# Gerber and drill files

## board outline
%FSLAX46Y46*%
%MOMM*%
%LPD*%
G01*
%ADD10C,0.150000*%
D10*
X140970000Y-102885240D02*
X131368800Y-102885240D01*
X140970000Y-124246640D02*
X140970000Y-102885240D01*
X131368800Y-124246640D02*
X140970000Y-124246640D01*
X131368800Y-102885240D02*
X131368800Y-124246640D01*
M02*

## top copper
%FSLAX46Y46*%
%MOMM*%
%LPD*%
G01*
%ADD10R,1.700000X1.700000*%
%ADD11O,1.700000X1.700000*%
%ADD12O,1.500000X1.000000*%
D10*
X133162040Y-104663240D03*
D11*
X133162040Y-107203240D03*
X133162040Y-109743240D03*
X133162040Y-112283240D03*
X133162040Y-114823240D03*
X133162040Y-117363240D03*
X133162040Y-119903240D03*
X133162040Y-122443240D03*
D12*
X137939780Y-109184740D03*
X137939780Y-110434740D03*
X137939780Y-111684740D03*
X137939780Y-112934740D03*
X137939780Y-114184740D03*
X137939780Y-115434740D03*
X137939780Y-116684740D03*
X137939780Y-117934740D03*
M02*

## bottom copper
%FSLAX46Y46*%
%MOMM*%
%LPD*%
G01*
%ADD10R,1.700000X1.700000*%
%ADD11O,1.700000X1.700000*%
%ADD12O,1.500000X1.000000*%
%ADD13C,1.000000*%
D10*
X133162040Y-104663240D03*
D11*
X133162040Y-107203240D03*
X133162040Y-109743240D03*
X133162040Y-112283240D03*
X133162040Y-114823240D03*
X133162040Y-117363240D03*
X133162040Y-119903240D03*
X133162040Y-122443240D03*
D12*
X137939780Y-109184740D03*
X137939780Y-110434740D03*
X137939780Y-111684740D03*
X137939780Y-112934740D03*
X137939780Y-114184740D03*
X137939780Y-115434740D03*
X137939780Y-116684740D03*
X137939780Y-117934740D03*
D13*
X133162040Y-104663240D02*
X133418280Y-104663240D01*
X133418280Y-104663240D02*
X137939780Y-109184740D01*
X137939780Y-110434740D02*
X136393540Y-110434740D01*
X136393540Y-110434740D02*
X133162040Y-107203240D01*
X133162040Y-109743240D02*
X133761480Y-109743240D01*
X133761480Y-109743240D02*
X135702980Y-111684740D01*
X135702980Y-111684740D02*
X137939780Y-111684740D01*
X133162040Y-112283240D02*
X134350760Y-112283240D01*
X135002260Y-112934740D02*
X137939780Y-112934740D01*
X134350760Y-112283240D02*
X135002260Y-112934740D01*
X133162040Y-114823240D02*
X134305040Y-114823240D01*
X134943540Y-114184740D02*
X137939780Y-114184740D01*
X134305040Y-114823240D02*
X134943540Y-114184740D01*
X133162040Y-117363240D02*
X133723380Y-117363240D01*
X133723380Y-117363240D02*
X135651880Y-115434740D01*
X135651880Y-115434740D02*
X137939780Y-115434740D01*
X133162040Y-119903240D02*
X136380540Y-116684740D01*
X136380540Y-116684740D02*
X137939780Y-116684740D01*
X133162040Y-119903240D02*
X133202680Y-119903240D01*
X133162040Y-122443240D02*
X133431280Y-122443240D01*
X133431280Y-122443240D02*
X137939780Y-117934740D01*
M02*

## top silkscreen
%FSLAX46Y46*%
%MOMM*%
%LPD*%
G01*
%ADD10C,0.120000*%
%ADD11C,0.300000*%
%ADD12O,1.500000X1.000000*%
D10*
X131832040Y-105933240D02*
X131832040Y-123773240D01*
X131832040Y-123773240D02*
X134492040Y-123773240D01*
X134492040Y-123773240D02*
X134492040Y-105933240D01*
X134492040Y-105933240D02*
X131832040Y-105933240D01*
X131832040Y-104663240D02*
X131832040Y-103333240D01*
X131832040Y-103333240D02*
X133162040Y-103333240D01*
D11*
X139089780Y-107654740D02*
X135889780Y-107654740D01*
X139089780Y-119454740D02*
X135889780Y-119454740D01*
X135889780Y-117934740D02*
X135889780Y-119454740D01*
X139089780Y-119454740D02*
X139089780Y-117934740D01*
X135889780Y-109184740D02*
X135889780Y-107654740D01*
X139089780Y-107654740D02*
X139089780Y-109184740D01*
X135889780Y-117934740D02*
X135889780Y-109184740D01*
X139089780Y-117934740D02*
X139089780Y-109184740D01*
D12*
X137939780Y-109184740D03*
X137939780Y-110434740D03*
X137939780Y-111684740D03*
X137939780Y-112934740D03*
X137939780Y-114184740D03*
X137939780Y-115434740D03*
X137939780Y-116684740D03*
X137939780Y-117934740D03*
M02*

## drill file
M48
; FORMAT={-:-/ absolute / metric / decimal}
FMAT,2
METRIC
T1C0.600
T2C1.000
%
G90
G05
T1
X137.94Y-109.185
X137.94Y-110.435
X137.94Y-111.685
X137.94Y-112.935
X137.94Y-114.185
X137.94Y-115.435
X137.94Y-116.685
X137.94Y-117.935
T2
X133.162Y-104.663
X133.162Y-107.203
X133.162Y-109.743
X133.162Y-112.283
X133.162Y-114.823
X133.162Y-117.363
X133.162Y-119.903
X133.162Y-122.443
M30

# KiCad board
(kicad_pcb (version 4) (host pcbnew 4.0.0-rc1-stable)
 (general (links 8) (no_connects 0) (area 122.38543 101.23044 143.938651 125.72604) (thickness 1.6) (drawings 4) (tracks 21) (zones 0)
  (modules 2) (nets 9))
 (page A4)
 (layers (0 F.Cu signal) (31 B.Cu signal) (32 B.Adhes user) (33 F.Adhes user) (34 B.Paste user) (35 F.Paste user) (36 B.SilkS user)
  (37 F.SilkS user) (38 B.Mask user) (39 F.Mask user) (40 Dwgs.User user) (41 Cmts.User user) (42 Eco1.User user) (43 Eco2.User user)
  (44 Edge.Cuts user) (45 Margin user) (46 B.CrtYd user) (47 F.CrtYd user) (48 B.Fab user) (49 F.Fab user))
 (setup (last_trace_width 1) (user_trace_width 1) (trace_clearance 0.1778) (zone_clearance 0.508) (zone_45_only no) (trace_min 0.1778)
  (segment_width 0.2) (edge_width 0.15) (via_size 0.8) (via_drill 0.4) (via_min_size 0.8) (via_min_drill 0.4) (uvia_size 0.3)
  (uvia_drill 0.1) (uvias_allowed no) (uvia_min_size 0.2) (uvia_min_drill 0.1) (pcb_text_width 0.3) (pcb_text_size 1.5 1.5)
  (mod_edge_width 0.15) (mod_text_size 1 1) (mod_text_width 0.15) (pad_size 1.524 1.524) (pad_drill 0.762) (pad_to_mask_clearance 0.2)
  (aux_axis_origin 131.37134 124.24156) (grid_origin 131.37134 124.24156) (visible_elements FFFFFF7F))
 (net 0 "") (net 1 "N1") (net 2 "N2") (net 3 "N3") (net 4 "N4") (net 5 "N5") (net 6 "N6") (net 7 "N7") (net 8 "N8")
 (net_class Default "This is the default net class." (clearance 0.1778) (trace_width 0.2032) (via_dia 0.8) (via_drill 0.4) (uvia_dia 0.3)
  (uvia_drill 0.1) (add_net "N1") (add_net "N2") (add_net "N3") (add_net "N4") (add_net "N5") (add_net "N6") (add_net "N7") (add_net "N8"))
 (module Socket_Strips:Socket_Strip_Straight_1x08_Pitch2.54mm (layer F.Cu) (at 133.16204 104.66324)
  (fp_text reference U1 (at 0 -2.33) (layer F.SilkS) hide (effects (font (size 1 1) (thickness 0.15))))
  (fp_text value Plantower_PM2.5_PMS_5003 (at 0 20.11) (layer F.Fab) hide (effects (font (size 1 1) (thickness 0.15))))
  (fp_line (start -1.33 1.27) (end -1.33 19.11) (layer F.SilkS) (width 0.12))
  (fp_line (start -1.33 19.11) (end 1.33 19.11) (layer F.SilkS) (width 0.12))
  (fp_line (start 1.33 19.11) (end 1.33 1.27) (layer F.SilkS) (width 0.12))
  (fp_line (start 1.33 1.27) (end -1.33 1.27) (layer F.SilkS) (width 0.12))
  (fp_line (start -1.33 0) (end -1.33 -1.33) (layer F.SilkS) (width 0.12))
  (fp_line (start -1.33 -1.33) (end 0 -1.33) (layer F.SilkS) (width 0.12))
  (pad 1 thru_hole rect (at 0 0) (size 1.7 1.7) (drill 1) (layers *.Cu *.Mask) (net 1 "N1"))
  (pad 2 thru_hole oval (at 0 2.54) (size 1.7 1.7) (drill 1) (layers *.Cu *.Mask) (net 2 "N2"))
  (pad 3 thru_hole oval (at 0 5.08) (size 1.7 1.7) (drill 1) (layers *.Cu *.Mask) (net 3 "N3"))
  (pad 4 thru_hole oval (at 0 7.62) (size 1.7 1.7) (drill 1) (layers *.Cu *.Mask) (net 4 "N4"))
  (pad 5 thru_hole oval (at 0 10.16) (size 1.7 1.7) (drill 1) (layers *.Cu *.Mask) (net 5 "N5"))
  (pad 6 thru_hole oval (at 0 12.7) (size 1.7 1.7) (drill 1) (layers *.Cu *.Mask) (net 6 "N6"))
  (pad 7 thru_hole oval (at 0 15.24) (size 1.7 1.7) (drill 1) (layers *.Cu *.Mask) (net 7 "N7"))
  (pad 8 thru_hole oval (at 0 17.78) (size 1.7 1.7) (drill 1) (layers *.Cu *.Mask) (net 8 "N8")))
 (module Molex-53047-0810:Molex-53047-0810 (layer F.Cu) (at 137.93978 117.93474 90)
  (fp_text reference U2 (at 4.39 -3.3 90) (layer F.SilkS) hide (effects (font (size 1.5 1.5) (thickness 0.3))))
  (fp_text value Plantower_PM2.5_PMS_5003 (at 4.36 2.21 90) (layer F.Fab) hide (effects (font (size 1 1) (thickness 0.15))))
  (fp_line (start 10.28 1.15) (end 10.28 -2.05) (layer F.SilkS) (width 0.3))
  (fp_line (start -1.52 1.15) (end -1.52 -2.05) (layer F.SilkS) (width 0.3))
  (fp_line (start 0 -2.05) (end -1.52 -2.05) (layer F.SilkS) (width 0.3))
  (fp_line (start -1.52 1.15) (end 0 1.15) (layer F.SilkS) (width 0.3))
  (fp_line (start 8.75 -2.05) (end 10.28 -2.05) (layer F.SilkS) (width 0.3))
  (fp_line (start 10.28 1.15) (end 8.75 1.15) (layer F.SilkS) (width 0.3))
  (fp_line (start 0 -2.05) (end 8.75 -2.05) (layer F.SilkS) (width 0.3))
  (fp_line (start 0 1.15) (end 8.75 1.15) (layer F.SilkS) (width 0.3))
  (pad 1 thru_hole oval (at 8.75 0 90) (size 1 1.5) (drill 0.6) (layers *.Cu *.Mask F.SilkS) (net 1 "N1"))
  (pad 2 thru_hole oval (at 7.5 0 90) (size 1 1.5) (drill 0.6) (layers *.Cu *.Mask F.SilkS) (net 2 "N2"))
  (pad 3 thru_hole oval (at 6.25 0 90) (size 1 1.5) (drill 0.6) (layers *.Cu *.Mask F.SilkS) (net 3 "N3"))
  (pad 4 thru_hole oval (at 5 0 90) (size 1 1.5) (drill 0.6) (layers *.Cu *.Mask F.SilkS) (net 4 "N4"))
  (pad 5 thru_hole oval (at 3.75 0 90) (size 1 1.5) (drill 0.6) (layers *.Cu *.Mask F.SilkS) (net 5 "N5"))
  (pad 6 thru_hole oval (at 2.5 0 90) (size 1 1.5) (drill 0.6) (layers *.Cu *.Mask F.SilkS) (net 6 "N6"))
  (pad 7 thru_hole oval (at 1.25 0 90) (size 1 1.5) (drill 0.6) (layers *.Cu *.Mask F.SilkS) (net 7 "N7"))
  (pad 8 thru_hole oval (at 0 0 90) (size 1 1.5) (drill 0.6) (layers *.Cu *.Mask F.SilkS) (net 8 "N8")))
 (gr_line (start 140.97 102.88524) (end 131.3688 102.88524) (angle 90) (layer Edge.Cuts) (width 0.15))
 (gr_line (start 140.97 124.24664) (end 140.97 102.88524) (angle 90) (layer Edge.Cuts) (width 0.15))
 (gr_line (start 131.3688 124.24664) (end 140.97 124.24664) (angle 90) (layer Edge.Cuts) (width 0.15))
 (gr_line (start 131.3688 102.88524) (end 131.3688 124.24664) (angle 90) (layer Edge.Cuts) (width 0.15))
 (segment (start 133.16204 104.66324) (end 133.41828 104.66324) (width 1) (layer B.Cu) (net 1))
 (segment (start 133.41828 104.66324) (end 137.93978 109.18474) (width 1) (layer B.Cu) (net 1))
 (segment (start 137.93978 110.43474) (end 136.39354 110.43474) (width 1) (layer B.Cu) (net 2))
 (segment (start 136.39354 110.43474) (end 133.16204 107.20324) (width 1) (layer B.Cu) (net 2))
 (segment (start 133.16204 109.74324) (end 133.76148 109.74324) (width 1) (layer B.Cu) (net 3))
 (segment (start 133.76148 109.74324) (end 135.70298 111.68474) (width 1) (layer B.Cu) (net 3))
 (segment (start 135.70298 111.68474) (end 137.93978 111.68474) (width 1) (layer B.Cu) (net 3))
 (segment (start 133.16204 112.28324) (end 134.35076 112.28324) (width 1) (layer B.Cu) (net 4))
 (segment (start 135.00226 112.93474) (end 137.93978 112.93474) (width 1) (layer B.Cu) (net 4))
 (segment (start 134.35076 112.28324) (end 135.00226 112.93474) (width 1) (layer B.Cu) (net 4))
 (segment (start 133.16204 114.82324) (end 134.30504 114.82324) (width 1) (layer B.Cu) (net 5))
 (segment (start 134.94354 114.18474) (end 137.93978 114.18474) (width 1) (layer B.Cu) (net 5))
 (segment (start 134.30504 114.82324) (end 134.94354 114.18474) (width 1) (layer B.Cu) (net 5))
 (segment (start 133.16204 117.36324) (end 133.72338 117.36324) (width 1) (layer B.Cu) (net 6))
 (segment (start 133.72338 117.36324) (end 135.65188 115.43474) (width 1) (layer B.Cu) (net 6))
 (segment (start 135.65188 115.43474) (end 137.93978 115.43474) (width 1) (layer B.Cu) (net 6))
 (segment (start 133.16204 119.90324) (end 136.38054 116.68474) (width 1) (layer B.Cu) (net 7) (status 400000))
 (segment (start 136.38054 116.68474) (end 137.93978 116.68474) (width 1) (layer B.Cu) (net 7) (status 800000))
 (segment (start 133.16204 119.90324) (end 133.20268 119.90324) (width 1) (layer B.Cu) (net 7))
 (segment (start 133.16204 122.44324) (end 133.43128 122.44324) (width 1) (layer B.Cu) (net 8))
 (segment (start 133.43128 122.44324) (end 137.93978 117.93474) (width 1) (layer B.Cu) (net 8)))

